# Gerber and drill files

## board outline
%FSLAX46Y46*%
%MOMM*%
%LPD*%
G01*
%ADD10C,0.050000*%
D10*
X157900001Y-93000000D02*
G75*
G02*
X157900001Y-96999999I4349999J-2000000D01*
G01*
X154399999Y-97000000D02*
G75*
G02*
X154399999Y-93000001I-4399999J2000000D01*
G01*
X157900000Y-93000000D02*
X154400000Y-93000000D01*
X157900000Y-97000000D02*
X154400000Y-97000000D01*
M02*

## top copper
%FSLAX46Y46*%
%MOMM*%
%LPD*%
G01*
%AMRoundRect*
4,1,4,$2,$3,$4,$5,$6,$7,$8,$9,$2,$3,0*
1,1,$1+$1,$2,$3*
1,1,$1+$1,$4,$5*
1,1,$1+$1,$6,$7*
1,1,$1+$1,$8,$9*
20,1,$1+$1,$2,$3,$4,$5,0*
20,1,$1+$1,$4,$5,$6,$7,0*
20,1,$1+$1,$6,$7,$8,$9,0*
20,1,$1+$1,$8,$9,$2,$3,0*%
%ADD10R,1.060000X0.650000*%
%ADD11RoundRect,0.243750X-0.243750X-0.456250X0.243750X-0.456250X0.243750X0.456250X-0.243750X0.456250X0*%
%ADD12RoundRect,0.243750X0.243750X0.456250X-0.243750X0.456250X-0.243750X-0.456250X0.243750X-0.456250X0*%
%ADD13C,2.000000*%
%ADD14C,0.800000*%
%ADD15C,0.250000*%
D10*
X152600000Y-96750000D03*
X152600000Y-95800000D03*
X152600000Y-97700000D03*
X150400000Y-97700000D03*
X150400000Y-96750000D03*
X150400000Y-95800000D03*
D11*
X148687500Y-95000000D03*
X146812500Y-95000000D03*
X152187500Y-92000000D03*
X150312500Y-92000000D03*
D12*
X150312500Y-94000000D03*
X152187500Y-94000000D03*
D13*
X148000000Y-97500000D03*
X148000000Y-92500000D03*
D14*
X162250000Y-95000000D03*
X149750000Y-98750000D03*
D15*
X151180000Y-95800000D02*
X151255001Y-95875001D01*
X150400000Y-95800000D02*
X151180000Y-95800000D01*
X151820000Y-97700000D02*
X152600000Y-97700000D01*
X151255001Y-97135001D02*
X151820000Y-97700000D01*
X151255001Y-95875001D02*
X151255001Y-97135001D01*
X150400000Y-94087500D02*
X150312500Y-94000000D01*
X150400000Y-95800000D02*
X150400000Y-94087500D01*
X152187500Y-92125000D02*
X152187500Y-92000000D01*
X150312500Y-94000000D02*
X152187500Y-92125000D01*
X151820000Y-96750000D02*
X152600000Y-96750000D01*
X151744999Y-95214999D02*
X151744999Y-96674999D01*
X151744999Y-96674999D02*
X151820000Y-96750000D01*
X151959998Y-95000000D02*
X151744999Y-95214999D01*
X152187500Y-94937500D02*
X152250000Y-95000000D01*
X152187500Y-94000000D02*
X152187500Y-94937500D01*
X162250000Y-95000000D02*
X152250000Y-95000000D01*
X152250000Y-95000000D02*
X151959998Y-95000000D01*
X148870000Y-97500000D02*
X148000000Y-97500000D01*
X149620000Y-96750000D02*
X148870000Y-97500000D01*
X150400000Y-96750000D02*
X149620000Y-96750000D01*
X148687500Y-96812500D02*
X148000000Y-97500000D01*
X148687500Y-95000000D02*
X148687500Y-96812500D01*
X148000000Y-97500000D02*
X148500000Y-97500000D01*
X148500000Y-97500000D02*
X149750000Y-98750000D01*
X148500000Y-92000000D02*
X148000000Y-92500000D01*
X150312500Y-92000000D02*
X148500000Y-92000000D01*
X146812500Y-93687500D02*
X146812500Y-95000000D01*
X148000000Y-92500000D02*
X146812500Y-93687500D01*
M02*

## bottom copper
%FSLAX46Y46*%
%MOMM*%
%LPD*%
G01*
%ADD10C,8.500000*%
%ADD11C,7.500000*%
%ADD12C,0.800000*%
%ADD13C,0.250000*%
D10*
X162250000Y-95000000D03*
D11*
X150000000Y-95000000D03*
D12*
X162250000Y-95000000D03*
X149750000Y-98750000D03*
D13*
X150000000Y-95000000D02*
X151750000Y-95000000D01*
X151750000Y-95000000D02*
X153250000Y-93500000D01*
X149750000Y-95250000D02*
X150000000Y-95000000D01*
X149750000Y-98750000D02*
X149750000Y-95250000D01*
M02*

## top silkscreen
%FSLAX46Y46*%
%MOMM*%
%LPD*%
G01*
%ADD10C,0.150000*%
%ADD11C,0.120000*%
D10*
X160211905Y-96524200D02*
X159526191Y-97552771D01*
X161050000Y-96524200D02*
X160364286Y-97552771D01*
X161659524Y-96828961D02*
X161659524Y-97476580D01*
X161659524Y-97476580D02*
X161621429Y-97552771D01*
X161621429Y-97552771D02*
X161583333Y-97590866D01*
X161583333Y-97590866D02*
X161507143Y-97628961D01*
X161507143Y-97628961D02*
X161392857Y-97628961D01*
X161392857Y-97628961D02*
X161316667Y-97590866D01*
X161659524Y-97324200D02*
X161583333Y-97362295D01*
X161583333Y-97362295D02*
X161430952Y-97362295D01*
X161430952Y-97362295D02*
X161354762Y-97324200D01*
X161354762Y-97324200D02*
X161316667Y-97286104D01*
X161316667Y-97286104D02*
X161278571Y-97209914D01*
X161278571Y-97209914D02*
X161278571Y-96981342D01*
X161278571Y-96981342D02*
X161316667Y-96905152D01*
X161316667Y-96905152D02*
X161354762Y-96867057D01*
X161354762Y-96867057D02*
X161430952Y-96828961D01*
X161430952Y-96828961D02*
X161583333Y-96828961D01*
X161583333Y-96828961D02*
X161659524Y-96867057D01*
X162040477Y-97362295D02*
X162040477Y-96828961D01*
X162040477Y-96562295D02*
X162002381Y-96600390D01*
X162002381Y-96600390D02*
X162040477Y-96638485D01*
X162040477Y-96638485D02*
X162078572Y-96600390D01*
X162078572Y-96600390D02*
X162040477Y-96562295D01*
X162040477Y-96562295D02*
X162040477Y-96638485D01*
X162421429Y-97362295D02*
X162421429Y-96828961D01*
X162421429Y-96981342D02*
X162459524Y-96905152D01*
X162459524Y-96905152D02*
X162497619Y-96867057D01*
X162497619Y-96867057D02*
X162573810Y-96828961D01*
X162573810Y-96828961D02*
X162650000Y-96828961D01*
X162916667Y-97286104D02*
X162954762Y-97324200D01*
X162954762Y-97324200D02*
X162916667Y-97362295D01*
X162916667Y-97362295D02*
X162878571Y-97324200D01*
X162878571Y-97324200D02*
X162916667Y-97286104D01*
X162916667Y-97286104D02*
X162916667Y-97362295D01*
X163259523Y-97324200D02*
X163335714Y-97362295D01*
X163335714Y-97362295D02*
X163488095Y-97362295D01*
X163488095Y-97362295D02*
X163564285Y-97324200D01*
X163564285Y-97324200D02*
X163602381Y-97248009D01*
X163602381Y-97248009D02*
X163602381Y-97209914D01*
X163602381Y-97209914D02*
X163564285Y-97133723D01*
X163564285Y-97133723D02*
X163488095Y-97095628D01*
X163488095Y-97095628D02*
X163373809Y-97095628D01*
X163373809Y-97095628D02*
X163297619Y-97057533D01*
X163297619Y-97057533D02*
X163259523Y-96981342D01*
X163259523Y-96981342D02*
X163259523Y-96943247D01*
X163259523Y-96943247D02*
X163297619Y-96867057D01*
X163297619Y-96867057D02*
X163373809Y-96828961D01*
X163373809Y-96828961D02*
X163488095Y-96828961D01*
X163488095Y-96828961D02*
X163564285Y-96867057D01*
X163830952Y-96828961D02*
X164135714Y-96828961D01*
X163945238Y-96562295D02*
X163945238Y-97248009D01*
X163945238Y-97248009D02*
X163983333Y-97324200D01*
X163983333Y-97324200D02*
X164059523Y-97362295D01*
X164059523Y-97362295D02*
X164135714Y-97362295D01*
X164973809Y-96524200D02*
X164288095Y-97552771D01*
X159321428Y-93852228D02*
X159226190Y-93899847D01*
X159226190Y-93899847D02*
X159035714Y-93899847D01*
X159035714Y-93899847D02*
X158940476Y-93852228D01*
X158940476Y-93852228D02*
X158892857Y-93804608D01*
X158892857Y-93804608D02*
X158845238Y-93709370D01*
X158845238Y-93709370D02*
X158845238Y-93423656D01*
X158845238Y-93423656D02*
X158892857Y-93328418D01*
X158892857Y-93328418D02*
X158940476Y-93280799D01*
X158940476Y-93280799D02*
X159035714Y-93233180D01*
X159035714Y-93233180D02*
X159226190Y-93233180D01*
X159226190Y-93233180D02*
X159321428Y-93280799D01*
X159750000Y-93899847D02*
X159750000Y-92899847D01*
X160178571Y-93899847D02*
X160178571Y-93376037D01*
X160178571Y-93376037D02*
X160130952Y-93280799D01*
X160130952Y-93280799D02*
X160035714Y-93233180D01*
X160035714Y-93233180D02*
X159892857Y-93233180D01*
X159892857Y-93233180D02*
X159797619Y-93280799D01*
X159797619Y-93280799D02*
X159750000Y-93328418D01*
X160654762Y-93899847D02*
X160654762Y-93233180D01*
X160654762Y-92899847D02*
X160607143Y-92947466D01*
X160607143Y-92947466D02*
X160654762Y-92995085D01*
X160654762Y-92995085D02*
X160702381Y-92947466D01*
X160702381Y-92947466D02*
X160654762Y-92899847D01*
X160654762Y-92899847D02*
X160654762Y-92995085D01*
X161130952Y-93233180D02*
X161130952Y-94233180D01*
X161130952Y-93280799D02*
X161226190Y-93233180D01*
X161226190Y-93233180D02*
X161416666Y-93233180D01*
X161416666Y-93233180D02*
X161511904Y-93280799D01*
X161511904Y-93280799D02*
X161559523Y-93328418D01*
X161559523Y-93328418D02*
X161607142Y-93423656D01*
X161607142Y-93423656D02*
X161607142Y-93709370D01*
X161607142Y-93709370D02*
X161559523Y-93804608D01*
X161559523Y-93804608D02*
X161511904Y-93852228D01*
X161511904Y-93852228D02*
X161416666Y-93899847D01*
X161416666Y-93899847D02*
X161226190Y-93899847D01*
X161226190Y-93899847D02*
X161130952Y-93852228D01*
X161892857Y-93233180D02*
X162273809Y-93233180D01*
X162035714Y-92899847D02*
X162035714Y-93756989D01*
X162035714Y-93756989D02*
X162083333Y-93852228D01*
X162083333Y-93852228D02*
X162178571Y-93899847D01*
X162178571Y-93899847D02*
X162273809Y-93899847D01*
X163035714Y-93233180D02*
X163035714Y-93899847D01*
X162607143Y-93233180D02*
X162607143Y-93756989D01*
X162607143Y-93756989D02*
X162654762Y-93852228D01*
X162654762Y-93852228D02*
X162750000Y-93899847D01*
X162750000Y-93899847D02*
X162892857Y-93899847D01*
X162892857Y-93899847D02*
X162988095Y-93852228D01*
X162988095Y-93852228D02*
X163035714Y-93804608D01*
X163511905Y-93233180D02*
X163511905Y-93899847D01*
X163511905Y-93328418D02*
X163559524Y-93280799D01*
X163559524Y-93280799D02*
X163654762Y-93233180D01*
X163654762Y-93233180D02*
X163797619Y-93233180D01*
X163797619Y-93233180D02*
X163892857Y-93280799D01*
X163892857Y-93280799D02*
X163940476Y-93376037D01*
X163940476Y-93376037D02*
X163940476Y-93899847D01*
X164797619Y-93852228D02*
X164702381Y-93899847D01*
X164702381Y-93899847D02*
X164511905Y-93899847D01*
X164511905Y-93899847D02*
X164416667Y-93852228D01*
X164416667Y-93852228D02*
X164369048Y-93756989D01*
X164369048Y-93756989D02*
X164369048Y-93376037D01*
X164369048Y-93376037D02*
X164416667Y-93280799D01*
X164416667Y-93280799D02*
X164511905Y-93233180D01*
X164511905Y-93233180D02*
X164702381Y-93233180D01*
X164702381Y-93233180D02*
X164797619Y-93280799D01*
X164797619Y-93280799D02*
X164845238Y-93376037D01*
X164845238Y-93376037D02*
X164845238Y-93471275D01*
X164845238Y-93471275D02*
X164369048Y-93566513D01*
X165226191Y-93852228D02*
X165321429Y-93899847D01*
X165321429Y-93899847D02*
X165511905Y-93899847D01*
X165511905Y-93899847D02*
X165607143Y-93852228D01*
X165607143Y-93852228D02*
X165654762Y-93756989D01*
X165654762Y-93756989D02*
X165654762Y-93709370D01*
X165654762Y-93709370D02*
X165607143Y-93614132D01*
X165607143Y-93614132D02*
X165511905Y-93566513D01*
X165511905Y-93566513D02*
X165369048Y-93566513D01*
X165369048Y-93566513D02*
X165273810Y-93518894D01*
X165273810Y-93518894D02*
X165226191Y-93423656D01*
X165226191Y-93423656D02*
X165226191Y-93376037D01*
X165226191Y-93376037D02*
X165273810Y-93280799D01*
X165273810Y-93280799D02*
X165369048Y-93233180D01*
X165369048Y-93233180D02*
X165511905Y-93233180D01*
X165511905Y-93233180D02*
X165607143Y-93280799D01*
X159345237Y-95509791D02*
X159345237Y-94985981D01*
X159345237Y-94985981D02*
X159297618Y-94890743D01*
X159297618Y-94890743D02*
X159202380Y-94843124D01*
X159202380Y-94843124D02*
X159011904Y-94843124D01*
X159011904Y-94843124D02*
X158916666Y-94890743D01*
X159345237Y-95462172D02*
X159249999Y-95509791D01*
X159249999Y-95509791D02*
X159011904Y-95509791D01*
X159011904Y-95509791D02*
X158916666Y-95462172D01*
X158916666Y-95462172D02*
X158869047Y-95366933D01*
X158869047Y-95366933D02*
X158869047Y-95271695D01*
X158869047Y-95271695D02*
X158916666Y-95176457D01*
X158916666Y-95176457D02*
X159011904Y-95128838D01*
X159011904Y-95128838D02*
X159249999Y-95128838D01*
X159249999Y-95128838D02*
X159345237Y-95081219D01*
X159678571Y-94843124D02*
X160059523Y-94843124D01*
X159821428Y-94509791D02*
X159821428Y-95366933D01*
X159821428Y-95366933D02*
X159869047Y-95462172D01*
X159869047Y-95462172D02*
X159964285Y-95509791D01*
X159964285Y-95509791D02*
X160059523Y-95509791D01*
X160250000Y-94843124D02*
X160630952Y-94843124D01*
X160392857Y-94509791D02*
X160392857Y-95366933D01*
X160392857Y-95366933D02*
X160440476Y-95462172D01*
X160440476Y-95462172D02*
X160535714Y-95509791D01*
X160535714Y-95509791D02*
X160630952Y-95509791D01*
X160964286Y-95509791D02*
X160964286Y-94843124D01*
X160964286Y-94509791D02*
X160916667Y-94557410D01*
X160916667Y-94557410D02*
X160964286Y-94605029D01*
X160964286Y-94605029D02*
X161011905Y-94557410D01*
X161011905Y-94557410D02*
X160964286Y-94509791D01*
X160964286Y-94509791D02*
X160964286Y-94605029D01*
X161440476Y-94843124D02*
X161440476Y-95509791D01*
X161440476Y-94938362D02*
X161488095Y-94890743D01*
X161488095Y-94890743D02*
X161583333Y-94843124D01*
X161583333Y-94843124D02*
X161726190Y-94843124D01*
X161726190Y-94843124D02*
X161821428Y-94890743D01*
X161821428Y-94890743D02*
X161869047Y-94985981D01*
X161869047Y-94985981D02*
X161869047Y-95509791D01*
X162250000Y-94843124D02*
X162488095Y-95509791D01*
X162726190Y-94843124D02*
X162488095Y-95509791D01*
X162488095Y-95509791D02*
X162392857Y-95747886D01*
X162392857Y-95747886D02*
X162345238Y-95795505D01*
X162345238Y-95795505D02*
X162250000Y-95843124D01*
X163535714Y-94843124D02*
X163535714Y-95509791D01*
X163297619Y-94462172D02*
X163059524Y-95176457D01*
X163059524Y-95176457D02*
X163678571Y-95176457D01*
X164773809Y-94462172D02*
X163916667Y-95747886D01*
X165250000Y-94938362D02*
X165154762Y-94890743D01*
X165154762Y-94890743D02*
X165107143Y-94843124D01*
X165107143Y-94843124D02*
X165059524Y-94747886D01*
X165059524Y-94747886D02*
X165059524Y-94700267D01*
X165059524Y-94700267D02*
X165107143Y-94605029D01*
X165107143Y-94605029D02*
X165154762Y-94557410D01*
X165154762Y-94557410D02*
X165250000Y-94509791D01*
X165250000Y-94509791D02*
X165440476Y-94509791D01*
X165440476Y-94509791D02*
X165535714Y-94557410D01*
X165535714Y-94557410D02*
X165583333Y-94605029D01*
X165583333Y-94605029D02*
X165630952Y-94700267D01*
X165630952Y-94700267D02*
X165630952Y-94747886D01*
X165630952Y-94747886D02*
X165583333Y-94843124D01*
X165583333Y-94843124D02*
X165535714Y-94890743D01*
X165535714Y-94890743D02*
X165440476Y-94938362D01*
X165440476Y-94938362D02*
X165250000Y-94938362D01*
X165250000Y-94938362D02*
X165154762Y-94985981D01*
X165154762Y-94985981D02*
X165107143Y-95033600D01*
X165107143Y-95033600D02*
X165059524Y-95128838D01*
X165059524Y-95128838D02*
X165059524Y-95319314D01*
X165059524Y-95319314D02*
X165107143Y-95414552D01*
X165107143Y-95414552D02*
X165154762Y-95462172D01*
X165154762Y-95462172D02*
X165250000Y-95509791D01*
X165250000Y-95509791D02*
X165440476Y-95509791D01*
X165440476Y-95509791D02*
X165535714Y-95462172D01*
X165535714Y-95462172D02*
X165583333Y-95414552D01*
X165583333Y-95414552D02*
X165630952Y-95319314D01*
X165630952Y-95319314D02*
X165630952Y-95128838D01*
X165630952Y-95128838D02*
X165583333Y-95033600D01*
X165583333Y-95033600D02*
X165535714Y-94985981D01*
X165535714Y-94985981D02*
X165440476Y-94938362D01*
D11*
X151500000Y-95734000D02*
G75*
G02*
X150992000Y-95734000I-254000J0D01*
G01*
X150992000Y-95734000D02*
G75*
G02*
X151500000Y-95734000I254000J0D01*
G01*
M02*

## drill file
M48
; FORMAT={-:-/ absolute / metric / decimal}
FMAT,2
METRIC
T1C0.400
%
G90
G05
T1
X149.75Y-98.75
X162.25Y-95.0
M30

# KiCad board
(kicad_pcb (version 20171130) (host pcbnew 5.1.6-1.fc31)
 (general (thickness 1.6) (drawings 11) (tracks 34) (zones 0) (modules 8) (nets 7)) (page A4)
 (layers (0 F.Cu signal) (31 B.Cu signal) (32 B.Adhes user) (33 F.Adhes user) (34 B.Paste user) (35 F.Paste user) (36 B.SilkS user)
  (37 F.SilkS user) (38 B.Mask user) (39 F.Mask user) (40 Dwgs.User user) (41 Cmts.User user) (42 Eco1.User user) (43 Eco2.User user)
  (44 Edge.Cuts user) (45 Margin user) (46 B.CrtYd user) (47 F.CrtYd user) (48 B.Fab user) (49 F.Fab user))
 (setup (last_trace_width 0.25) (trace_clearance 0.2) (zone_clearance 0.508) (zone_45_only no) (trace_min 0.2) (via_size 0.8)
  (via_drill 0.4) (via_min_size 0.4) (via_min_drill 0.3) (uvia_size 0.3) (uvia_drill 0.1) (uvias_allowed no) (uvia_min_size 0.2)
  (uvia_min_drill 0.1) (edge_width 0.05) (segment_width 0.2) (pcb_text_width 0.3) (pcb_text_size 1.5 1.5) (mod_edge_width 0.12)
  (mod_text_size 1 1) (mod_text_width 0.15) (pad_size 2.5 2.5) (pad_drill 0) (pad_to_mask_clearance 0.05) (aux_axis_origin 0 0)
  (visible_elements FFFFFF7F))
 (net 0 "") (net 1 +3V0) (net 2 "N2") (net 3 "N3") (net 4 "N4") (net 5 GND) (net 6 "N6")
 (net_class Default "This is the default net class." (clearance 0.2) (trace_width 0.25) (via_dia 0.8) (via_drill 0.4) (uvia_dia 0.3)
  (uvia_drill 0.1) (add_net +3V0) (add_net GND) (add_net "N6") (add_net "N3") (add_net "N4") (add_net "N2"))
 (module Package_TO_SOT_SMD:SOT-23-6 (layer F.Cu) (at 151.5 96.75)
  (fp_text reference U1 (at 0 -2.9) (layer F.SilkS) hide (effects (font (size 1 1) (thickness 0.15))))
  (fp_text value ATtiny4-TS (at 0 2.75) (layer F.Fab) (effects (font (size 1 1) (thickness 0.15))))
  (fp_circle (center -0.254 -1.016) (end 0 -1.016) (layer F.SilkS) (width 0.12))
  (pad 5 smd rect (at 1.1 0) (size 1.06 0.65) (layers F.Cu F.Paste F.Mask) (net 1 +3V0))
  (pad 6 smd rect (at 1.1 -0.95) (size 1.06 0.65) (layers F.Cu F.Paste F.Mask) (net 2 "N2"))
  (pad 4 smd rect (at 1.1 0.95) (size 1.06 0.65) (layers F.Cu F.Paste F.Mask) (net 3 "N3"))
  (pad 3 smd rect (at -1.1 0.95) (size 1.06 0.65) (layers F.Cu F.Paste F.Mask) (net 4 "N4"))
  (pad 2 smd rect (at -1.1 0) (size 1.06 0.65) (layers F.Cu F.Paste F.Mask) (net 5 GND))
  (pad 1 smd rect (at -1.1 -0.95) (size 1.06 0.65) (layers F.Cu F.Paste F.Mask) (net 3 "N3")))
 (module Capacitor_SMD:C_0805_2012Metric (layer F.Cu) (at 147.75 95)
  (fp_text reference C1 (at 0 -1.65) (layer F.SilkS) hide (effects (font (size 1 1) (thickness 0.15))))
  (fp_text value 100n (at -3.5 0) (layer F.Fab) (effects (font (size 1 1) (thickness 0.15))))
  (pad 2 smd roundrect (at 0.9375 0) (size 0.975 1.4) (layers F.Cu F.Paste F.Mask) (roundrect_rratio 0.25) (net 5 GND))
  (pad 1 smd roundrect (at -0.9375 0) (size 0.975 1.4) (layers F.Cu F.Paste F.Mask) (roundrect_rratio 0.25) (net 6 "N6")))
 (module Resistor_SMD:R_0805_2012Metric (layer F.Cu) (at 151.25 92)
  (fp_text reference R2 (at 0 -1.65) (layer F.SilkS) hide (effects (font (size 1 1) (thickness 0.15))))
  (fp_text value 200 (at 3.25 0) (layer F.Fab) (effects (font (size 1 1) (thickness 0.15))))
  (pad 2 smd roundrect (at 0.9375 0) (size 0.975 1.4) (layers F.Cu F.Paste F.Mask) (roundrect_rratio 0.25) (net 3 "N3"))
  (pad 1 smd roundrect (at -0.9375 0) (size 0.975 1.4) (layers F.Cu F.Paste F.Mask) (roundrect_rratio 0.25) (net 6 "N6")))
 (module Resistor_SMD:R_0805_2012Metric (layer F.Cu) (at 151.25 94 180)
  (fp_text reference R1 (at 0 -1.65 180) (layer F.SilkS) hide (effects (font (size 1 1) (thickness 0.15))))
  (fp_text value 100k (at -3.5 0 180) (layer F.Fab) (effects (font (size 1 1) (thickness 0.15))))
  (pad 2 smd roundrect (at 0.9375 0 180) (size 0.975 1.4) (layers F.Cu F.Paste F.Mask) (roundrect_rratio 0.25) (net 3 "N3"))
  (pad 1 smd roundrect (at -0.9375 0 180) (size 0.975 1.4) (layers F.Cu F.Paste F.Mask) (roundrect_rratio 0.25) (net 1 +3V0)))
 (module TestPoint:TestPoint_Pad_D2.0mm (layer F.Cu) (at 148 97.5 180)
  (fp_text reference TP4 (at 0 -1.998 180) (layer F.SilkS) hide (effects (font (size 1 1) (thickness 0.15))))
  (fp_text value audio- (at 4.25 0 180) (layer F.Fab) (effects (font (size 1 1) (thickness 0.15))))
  (pad 1 smd circle (at 0 0 180) (size 2 2) (layers F.Cu F.Mask) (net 5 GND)))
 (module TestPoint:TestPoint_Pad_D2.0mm (layer F.Cu) (at 148 92.5 180)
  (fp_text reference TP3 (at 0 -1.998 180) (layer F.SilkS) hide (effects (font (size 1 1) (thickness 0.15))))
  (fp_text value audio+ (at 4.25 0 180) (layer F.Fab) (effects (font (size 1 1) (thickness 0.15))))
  (pad 1 smd circle (at 0 0 180) (size 2 2) (layers F.Cu F.Mask) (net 6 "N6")))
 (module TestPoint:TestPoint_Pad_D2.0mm (layer B.Cu) (at 162.25 95)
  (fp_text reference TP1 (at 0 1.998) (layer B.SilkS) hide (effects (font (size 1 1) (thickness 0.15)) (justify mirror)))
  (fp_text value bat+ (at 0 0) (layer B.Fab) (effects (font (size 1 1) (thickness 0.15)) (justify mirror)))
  (pad 1 smd circle (at 0 0) (size 8.5 8.5) (layers B.Cu B.Mask) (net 1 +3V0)))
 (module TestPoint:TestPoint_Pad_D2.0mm (layer B.Cu) (at 150 95)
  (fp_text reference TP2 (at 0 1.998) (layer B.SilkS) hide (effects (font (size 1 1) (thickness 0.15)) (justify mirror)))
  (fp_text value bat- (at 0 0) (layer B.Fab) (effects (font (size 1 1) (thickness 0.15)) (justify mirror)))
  (pad 1 smd circle (at 0 0) (size 7.5 7.5) (layers B.Cu B.Mask) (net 5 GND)))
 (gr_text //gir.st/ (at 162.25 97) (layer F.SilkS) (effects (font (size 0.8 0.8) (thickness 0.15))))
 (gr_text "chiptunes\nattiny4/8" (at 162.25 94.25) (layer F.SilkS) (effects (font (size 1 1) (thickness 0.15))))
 (gr_arc (start 162.25 95) (end 157.900001 96.999999) (angle -310.6168837) (layer Edge.Cuts) (width 0.05))
 (gr_arc (start 150 95) (end 154.399999 93.000001) (angle -311.1120904) (layer Edge.Cuts) (width 0.05))
 (gr_line (start 157.9 93) (end 154.4 93) (layer Edge.Cuts) (width 0.05))
 (gr_line (start 157.9 97) (end 154.4 97) (layer Edge.Cuts) (width 0.05))
 (segment (start 151.18 95.8) (end 151.255001 95.875001) (width 0.25) (layer F.Cu) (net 3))
 (segment (start 150.4 95.8) (end 151.18 95.8) (width 0.25) (layer F.Cu) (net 3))
 (segment (start 151.82 97.7) (end 152.6 97.7) (width 0.25) (layer F.Cu) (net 3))
 (segment (start 151.255001 97.135001) (end 151.82 97.7) (width 0.25) (layer F.Cu) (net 3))
 (segment (start 151.255001 95.875001) (end 151.255001 97.135001) (width 0.25) (layer F.Cu) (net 3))
 (segment (start 150.4 94.0875) (end 150.3125 94) (width 0.25) (layer F.Cu) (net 3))
 (segment (start 150.4 95.8) (end 150.4 94.0875) (width 0.25) (layer F.Cu) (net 3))
 (segment (start 152.1875 92.125) (end 152.1875 92) (width 0.25) (layer F.Cu) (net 3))
 (segment (start 150.3125 94) (end 152.1875 92.125) (width 0.25) (layer F.Cu) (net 3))
 (via (at 162.25 95) (size 0.8) (drill 0.4) (layers F.Cu B.Cu) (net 1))
 (segment (start 151.82 96.75) (end 152.6 96.75) (width 0.25) (layer F.Cu) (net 1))
 (segment (start 151.744999 95.214999) (end 151.744999 96.674999) (width 0.25) (layer F.Cu) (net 1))
 (segment (start 151.744999 96.674999) (end 151.82 96.75) (width 0.25) (layer F.Cu) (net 1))
 (segment (start 151.959998 95) (end 151.744999 95.214999) (width 0.25) (layer F.Cu) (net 1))
 (segment (start 152.1875 94.9375) (end 152.25 95) (width 0.25) (layer F.Cu) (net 1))
 (segment (start 152.1875 94) (end 152.1875 94.9375) (width 0.25) (layer F.Cu) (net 1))
 (segment (start 162.25 95) (end 152.25 95) (width 0.25) (layer F.Cu) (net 1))
 (segment (start 152.25 95) (end 151.959998 95) (width 0.25) (layer F.Cu) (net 1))
 (segment (start 150 95) (end 151.75 95) (width 0.25) (layer B.Cu) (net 5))
 (segment (start 151.75 95) (end 153.25 93.5) (width 0.25) (layer B.Cu) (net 5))
 (segment (start 148.87 97.5) (end 148 97.5) (width 0.25) (layer F.Cu) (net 5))
 (segment (start 149.62 96.75) (end 148.87 97.5) (width 0.25) (layer F.Cu) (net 5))
 (segment (start 150.4 96.75) (end 149.62 96.75) (width 0.25) (layer F.Cu) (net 5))
 (segment (start 148.6875 96.8125) (end 148 97.5) (width 0.25) (layer F.Cu) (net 5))
 (segment (start 148.6875 95) (end 148.6875 96.8125) (width 0.25) (layer F.Cu) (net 5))
 (via (at 149.75 98.75) (size 0.8) (drill 0.4) (layers F.Cu B.Cu) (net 5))
 (segment (start 148 97.5) (end 148.5 97.5) (width 0.25) (layer F.Cu) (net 5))
 (segment (start 148.5 97.5) (end 149.75 98.75) (width 0.25) (layer F.Cu) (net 5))
 (segment (start 149.75 95.25) (end 150 95) (width 0.25) (layer B.Cu) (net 5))
 (segment (start 149.75 98.75) (end 149.75 95.25) (width 0.25) (layer B.Cu) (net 5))
 (segment (start 148.5 92) (end 148 92.5) (width 0.25) (layer F.Cu) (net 6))
 (segment (start 150.3125 92) (end 148.5 92) (width 0.25) (layer F.Cu) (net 6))
 (segment (start 146.8125 93.6875) (end 146.8125 95) (width 0.25) (layer F.Cu) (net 6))
 (segment (start 148 92.5) (end 146.8125 93.6875) (width 0.25) (layer F.Cu) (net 6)))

